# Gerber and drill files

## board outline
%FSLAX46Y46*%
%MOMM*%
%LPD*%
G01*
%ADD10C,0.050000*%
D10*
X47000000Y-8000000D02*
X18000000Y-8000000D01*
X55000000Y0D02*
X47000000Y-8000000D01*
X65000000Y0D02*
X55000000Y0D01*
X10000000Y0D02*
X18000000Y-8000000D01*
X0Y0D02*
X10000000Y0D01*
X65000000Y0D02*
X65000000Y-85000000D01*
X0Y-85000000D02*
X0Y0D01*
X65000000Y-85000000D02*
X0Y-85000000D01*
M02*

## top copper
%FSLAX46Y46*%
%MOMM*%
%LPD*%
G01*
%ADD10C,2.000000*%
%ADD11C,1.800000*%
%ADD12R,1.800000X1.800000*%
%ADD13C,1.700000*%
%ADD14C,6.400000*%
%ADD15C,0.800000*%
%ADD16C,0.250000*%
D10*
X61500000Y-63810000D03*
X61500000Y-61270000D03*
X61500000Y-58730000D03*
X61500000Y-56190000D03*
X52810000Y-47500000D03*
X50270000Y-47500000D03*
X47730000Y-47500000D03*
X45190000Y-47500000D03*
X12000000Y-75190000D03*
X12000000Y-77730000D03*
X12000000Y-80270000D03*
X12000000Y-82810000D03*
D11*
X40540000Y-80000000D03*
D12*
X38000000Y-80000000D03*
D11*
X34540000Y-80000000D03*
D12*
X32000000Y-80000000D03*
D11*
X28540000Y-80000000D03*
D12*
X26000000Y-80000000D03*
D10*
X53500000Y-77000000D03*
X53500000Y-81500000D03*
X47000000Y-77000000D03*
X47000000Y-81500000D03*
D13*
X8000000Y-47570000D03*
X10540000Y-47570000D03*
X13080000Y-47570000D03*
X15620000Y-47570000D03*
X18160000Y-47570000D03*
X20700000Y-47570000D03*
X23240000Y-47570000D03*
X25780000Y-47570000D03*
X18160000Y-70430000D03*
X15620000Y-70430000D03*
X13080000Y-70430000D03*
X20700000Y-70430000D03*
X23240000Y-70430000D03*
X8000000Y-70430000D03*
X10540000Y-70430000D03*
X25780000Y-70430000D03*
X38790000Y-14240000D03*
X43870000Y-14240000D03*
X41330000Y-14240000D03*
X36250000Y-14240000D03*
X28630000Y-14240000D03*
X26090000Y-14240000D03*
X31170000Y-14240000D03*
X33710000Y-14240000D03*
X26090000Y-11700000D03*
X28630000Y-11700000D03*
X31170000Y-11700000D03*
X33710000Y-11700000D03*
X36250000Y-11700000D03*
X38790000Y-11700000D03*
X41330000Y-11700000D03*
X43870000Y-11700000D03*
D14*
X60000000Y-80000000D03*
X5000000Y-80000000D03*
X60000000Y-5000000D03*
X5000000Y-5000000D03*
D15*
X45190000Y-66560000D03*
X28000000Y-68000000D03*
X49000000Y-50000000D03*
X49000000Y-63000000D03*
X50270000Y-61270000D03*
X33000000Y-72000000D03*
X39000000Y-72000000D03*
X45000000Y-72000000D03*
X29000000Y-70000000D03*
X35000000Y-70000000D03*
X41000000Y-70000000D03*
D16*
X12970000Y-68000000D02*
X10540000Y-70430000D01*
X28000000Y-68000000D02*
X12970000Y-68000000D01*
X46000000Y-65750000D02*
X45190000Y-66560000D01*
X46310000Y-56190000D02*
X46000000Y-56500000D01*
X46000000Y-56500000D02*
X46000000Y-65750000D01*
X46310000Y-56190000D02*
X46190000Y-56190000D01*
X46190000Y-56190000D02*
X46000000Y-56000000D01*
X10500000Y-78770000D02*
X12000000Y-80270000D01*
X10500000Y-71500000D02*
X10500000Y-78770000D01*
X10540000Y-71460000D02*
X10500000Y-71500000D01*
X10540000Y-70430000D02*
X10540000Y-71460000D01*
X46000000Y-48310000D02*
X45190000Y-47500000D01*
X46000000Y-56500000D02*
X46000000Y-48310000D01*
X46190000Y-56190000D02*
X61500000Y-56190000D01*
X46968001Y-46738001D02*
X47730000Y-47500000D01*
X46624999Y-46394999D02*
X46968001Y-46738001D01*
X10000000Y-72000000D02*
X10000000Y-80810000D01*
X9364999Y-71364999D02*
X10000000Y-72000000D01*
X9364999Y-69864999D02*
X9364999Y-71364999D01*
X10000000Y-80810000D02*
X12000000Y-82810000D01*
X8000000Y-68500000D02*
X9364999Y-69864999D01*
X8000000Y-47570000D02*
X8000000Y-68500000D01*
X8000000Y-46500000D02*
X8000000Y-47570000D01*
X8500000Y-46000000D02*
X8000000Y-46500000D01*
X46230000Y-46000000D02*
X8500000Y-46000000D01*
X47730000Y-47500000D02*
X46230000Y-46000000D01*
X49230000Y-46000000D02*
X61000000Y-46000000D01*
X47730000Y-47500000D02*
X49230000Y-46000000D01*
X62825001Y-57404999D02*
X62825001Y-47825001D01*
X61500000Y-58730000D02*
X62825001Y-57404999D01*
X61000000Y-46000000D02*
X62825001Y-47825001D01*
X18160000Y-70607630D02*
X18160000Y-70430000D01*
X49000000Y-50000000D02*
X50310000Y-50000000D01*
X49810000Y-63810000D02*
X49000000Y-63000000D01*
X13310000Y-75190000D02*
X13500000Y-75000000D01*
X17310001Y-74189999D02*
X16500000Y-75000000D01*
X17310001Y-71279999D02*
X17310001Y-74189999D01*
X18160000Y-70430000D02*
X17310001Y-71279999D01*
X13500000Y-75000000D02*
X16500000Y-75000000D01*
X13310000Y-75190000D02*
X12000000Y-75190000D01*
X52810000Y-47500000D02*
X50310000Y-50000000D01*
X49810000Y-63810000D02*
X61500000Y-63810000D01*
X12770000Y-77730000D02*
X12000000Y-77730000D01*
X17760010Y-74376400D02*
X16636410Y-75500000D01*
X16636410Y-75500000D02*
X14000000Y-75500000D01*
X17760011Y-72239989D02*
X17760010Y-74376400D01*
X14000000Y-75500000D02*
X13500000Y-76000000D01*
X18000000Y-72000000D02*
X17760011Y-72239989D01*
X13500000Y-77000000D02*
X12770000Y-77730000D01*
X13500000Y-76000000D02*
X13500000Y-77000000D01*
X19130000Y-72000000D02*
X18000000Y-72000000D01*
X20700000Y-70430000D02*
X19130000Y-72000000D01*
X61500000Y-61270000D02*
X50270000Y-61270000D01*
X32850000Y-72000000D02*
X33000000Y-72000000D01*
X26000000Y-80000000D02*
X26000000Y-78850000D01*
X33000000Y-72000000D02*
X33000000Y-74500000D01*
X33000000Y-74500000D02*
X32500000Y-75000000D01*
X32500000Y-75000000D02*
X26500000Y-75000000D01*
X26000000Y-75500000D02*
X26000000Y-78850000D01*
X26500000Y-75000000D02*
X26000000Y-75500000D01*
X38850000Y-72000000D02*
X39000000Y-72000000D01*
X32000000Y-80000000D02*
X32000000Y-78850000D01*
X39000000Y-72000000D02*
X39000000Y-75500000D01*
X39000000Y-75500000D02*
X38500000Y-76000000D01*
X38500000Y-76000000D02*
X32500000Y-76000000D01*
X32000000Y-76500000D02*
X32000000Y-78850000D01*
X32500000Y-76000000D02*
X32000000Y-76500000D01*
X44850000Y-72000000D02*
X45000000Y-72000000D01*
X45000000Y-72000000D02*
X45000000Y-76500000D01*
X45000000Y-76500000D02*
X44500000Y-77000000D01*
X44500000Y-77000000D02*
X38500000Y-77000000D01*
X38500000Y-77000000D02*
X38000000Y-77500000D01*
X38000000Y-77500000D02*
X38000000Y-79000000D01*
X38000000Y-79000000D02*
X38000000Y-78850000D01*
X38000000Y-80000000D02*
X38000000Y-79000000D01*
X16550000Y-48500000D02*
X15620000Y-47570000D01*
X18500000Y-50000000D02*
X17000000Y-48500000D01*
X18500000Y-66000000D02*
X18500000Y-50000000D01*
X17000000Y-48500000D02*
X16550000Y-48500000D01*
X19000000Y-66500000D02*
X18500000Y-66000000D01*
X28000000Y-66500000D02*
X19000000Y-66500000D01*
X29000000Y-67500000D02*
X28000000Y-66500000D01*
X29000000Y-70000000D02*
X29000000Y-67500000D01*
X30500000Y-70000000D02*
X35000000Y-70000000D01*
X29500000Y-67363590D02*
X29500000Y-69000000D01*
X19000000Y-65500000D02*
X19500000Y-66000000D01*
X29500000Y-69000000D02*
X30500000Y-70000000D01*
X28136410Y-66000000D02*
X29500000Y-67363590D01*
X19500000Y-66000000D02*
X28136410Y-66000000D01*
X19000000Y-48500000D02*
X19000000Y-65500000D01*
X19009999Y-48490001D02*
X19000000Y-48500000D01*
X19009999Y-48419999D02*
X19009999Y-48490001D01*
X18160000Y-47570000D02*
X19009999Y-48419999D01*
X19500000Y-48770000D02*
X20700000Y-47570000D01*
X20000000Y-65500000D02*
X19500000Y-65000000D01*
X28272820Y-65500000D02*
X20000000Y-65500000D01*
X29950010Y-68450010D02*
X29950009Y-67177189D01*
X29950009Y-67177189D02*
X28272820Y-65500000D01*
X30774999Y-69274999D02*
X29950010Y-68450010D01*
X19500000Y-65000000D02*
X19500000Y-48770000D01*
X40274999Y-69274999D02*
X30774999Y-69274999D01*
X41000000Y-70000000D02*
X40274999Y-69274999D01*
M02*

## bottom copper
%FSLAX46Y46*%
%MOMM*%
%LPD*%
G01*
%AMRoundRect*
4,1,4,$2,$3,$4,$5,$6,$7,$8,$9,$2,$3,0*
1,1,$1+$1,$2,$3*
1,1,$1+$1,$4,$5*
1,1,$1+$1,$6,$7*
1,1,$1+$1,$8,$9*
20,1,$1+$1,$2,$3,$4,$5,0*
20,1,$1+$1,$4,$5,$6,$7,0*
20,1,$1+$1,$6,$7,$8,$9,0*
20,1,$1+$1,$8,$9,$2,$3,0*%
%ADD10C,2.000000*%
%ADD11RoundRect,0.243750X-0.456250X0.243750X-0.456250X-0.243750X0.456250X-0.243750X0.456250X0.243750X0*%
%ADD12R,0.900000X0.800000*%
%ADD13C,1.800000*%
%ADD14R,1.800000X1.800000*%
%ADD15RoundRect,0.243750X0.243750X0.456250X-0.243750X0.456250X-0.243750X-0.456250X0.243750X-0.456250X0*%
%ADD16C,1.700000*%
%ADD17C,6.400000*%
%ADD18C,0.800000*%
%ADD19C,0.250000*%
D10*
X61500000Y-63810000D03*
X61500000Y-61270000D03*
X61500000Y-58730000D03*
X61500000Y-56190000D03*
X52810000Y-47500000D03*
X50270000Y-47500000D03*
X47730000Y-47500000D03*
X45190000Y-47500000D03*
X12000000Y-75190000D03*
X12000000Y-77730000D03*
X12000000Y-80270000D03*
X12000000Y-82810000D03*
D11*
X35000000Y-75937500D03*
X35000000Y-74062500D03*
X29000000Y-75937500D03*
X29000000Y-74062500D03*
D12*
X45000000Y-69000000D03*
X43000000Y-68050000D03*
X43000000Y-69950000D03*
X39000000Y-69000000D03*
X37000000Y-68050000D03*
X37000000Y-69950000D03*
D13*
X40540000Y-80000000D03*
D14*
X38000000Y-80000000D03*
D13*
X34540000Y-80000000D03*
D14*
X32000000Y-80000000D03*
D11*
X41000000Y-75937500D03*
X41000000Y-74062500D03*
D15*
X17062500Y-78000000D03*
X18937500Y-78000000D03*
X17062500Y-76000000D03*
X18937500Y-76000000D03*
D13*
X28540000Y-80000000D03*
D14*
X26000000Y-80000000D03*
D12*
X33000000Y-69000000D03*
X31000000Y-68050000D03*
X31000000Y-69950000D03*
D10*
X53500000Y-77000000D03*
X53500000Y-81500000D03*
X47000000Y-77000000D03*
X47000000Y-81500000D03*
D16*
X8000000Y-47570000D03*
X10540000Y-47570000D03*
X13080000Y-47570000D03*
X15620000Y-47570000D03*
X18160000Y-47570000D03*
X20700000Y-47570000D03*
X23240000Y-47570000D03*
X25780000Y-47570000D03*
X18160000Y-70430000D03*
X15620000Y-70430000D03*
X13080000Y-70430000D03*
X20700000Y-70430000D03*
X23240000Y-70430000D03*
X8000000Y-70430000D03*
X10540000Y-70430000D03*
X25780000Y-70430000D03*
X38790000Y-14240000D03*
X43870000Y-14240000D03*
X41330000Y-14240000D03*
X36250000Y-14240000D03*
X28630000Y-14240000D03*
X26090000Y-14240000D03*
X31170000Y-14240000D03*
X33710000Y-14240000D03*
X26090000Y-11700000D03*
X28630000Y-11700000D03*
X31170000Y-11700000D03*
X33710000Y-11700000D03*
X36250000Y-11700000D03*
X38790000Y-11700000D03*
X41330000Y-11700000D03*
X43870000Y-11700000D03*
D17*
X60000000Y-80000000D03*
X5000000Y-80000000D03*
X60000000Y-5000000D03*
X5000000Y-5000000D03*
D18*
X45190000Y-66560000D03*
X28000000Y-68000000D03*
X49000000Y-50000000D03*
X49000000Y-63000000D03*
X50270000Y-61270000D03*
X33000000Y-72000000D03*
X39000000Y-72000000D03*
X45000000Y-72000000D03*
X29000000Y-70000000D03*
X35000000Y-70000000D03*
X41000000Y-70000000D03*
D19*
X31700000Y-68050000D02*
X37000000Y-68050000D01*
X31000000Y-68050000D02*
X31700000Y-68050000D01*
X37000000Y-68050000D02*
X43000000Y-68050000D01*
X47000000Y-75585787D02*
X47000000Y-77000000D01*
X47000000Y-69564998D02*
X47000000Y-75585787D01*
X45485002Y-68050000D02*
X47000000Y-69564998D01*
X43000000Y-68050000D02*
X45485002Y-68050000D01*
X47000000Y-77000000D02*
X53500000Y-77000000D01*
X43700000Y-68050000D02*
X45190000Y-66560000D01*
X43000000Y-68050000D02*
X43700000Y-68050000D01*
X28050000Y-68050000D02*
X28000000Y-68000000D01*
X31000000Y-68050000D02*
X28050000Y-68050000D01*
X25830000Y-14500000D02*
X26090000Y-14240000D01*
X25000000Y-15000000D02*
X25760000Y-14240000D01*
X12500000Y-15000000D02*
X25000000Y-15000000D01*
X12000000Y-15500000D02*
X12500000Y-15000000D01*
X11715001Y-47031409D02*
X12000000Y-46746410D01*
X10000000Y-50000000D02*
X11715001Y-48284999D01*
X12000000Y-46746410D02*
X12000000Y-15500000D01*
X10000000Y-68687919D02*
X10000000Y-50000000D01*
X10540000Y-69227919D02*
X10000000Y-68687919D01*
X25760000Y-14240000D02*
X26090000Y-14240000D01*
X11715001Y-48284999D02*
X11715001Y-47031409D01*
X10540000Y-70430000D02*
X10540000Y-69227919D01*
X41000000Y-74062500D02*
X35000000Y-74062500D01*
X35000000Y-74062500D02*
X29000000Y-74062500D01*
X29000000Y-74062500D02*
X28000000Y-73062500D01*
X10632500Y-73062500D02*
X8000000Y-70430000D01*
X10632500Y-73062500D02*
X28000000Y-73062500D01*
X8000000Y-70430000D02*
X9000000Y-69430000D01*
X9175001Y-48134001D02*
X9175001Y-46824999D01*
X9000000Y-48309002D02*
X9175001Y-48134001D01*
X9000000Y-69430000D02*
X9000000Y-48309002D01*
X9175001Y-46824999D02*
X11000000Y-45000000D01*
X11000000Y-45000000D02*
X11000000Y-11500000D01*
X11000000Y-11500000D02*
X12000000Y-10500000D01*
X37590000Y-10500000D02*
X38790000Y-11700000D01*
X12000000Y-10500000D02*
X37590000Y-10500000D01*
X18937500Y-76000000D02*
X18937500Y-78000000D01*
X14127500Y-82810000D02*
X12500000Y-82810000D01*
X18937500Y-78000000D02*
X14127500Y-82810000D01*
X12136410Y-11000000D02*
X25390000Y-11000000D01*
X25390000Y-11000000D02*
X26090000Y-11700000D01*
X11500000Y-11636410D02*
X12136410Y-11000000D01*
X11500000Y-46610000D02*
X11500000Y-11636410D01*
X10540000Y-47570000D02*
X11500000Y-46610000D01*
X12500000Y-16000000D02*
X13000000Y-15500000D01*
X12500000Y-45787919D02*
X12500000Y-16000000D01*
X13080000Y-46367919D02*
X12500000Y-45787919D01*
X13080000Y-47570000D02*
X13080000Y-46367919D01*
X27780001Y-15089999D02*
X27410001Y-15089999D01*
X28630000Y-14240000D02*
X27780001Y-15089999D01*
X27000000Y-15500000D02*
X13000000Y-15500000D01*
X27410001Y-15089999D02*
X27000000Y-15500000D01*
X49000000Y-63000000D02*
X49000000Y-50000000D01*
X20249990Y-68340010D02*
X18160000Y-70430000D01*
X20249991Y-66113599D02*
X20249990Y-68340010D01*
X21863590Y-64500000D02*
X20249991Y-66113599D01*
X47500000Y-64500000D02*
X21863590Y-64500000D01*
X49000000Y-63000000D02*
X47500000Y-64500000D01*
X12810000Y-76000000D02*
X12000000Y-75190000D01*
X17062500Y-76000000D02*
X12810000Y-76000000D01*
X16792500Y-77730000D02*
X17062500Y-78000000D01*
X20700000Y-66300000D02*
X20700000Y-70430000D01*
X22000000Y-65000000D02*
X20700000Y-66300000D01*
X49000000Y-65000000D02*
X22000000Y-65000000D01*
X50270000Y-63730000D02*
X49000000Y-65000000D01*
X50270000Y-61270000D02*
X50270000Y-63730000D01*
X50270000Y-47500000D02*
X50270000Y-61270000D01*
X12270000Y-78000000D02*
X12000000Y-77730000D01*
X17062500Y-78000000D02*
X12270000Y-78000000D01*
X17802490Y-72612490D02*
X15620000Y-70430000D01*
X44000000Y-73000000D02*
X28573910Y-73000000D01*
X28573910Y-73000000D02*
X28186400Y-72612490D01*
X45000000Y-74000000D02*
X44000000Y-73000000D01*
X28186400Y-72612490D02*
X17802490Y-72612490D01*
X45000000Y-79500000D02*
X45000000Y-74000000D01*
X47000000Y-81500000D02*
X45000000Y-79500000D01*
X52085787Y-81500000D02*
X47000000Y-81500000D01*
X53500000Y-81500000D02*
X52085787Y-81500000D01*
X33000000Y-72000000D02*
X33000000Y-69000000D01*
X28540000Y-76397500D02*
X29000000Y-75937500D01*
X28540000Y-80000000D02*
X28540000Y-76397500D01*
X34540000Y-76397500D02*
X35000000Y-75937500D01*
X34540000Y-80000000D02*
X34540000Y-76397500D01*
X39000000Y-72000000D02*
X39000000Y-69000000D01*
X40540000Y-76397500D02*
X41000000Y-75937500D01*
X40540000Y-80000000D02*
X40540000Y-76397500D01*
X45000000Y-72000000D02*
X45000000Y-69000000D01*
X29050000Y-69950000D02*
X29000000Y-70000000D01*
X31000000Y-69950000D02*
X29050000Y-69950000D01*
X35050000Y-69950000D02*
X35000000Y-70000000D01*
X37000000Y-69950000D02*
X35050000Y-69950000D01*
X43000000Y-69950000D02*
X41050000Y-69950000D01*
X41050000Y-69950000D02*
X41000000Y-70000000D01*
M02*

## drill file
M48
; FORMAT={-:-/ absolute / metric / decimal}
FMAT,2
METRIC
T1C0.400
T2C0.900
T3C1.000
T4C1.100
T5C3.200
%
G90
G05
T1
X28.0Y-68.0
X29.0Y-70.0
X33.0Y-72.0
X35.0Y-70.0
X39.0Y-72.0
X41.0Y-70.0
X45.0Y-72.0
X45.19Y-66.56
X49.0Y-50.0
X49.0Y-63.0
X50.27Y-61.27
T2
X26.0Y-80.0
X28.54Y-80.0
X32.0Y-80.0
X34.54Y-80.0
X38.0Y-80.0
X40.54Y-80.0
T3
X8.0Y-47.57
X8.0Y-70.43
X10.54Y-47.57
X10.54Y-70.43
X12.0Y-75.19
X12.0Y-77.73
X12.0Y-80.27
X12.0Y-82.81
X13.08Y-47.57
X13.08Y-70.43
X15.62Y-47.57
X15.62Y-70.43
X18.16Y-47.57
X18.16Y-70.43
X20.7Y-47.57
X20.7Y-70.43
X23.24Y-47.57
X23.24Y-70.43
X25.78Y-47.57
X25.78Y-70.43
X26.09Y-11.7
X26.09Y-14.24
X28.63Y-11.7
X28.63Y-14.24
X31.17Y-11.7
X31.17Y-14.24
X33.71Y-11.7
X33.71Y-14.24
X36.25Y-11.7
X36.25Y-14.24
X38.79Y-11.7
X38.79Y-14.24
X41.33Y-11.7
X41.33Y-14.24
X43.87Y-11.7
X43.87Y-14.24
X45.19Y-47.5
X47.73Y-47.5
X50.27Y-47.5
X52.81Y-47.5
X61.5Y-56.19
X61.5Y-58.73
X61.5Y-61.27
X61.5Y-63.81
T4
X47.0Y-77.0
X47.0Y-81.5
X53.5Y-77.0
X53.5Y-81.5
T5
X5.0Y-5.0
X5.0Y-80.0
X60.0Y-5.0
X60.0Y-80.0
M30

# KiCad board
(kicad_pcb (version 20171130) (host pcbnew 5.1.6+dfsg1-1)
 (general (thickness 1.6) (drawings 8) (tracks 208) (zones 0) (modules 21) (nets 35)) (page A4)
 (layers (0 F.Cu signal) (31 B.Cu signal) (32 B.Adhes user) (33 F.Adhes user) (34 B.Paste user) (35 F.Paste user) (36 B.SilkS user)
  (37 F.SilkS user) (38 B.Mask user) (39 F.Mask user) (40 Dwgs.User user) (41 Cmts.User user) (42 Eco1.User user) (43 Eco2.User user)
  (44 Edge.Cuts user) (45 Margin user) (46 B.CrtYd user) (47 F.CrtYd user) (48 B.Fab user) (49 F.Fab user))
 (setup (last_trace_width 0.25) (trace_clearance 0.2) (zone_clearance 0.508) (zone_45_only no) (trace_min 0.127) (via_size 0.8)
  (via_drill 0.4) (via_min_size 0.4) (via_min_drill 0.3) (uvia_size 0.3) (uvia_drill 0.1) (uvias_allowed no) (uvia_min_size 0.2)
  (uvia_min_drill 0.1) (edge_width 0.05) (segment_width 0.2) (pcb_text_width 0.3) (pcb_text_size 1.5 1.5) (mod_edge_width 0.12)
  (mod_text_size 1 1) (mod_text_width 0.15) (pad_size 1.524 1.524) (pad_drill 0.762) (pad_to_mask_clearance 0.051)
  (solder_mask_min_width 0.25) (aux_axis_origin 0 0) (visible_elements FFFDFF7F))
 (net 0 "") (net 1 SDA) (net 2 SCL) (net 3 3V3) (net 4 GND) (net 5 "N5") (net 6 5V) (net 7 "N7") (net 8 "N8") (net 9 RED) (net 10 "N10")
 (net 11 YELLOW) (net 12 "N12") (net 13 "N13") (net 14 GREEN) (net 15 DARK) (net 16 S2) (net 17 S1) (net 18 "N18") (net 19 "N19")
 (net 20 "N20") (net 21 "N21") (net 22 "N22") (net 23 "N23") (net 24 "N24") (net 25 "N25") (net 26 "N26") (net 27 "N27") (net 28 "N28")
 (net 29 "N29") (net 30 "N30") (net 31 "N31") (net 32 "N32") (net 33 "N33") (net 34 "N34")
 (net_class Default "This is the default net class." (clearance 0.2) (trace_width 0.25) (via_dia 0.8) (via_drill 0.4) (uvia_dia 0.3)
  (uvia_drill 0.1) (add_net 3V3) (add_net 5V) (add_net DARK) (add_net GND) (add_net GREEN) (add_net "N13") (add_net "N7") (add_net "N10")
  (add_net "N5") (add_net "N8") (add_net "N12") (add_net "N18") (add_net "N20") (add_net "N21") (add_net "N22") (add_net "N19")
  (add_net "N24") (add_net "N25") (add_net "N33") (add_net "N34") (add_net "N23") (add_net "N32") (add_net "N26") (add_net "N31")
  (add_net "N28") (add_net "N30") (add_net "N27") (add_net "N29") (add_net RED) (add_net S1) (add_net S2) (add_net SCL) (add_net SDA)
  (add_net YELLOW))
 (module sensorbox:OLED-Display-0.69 (layer F.Cu) (at 49 60 270)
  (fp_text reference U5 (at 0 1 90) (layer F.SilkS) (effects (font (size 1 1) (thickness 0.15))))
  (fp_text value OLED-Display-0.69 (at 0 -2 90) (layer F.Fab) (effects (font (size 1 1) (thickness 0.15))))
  (pad 4 thru_hole circle (at 3.81 -12.5 270) (size 2 2) (drill 1) (layers *.Cu *.Mask) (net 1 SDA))
  (pad 3 thru_hole circle (at 1.27 -12.5 270) (size 2 2) (drill 1) (layers *.Cu *.Mask) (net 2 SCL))
  (pad 2 thru_hole circle (at -1.27 -12.5 270) (size 2 2) (drill 1) (layers *.Cu *.Mask) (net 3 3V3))
  (pad 1 thru_hole circle (at -3.81 -12.5 270) (size 2 2) (drill 1) (layers *.Cu *.Mask) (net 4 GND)))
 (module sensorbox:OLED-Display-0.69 (layer F.Cu) (at 49 60)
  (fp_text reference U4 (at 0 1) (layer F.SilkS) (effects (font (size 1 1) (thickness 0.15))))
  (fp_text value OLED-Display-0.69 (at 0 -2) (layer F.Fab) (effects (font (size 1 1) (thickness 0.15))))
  (pad 4 thru_hole circle (at 3.81 -12.5) (size 2 2) (drill 1) (layers *.Cu *.Mask) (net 1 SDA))
  (pad 3 thru_hole circle (at 1.27 -12.5) (size 2 2) (drill 1) (layers *.Cu *.Mask) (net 2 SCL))
  (pad 2 thru_hole circle (at -1.27 -12.5) (size 2 2) (drill 1) (layers *.Cu *.Mask) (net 3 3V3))
  (pad 1 thru_hole circle (at -3.81 -12.5) (size 2 2) (drill 1) (layers *.Cu *.Mask) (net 4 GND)))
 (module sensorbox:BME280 (layer F.Cu) (at 16.5 79 90)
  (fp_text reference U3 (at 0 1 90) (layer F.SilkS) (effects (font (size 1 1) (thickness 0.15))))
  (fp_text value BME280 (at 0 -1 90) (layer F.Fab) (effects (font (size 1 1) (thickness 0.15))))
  (pad 4 thru_hole circle (at 3.81 -4.5 90) (size 2 2) (drill 1) (layers *.Cu *.Mask) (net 1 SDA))
  (pad 3 thru_hole circle (at 1.27 -4.5 90) (size 2 2) (drill 1) (layers *.Cu *.Mask) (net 2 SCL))
  (pad 2 thru_hole circle (at -1.27 -4.5 90) (size 2 2) (drill 1) (layers *.Cu *.Mask) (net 4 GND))
  (pad 1 thru_hole circle (at -3.81 -4.5 90) (size 2 2) (drill 1) (layers *.Cu *.Mask) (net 3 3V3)))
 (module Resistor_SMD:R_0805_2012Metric (layer B.Cu) (at 35 75 270)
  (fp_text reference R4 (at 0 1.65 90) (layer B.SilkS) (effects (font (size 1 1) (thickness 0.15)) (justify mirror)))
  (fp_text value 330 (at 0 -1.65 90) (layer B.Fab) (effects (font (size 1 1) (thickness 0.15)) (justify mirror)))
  (pad 2 smd roundrect (at 0.9375 0 270) (size 0.975 1.4) (layers B.Cu B.Paste B.Mask) (roundrect_rratio 0.25) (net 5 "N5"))
  (pad 1 smd roundrect (at -0.9375 0 270) (size 0.975 1.4) (layers B.Cu B.Paste B.Mask) (roundrect_rratio 0.25) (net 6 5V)))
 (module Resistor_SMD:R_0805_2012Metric (layer B.Cu) (at 29 75 270)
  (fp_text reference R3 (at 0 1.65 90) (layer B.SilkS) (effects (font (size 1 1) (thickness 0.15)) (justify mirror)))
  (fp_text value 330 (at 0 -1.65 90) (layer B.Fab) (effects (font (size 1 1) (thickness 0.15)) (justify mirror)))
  (pad 2 smd roundrect (at 0.9375 0 270) (size 0.975 1.4) (layers B.Cu B.Paste B.Mask) (roundrect_rratio 0.25) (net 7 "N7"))
  (pad 1 smd roundrect (at -0.9375 0 270) (size 0.975 1.4) (layers B.Cu B.Paste B.Mask) (roundrect_rratio 0.25) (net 6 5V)))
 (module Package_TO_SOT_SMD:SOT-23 (layer B.Cu) (at 44 69)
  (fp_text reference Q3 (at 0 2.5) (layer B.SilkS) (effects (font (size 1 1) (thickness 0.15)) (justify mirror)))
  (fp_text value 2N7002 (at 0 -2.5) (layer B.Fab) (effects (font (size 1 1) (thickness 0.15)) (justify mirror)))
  (pad 3 smd rect (at 1 0) (size 0.9 0.8) (layers B.Cu B.Paste B.Mask) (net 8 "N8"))
  (pad 2 smd rect (at -1 -0.95) (size 0.9 0.8) (layers B.Cu B.Paste B.Mask) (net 4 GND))
  (pad 1 smd rect (at -1 0.95) (size 0.9 0.8) (layers B.Cu B.Paste B.Mask) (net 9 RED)))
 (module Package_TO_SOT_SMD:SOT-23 (layer B.Cu) (at 38 69)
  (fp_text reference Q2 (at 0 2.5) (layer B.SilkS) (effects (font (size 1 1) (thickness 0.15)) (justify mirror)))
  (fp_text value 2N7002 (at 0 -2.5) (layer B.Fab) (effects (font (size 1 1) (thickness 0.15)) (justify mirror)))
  (pad 3 smd rect (at 1 0) (size 0.9 0.8) (layers B.Cu B.Paste B.Mask) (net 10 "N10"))
  (pad 2 smd rect (at -1 -0.95) (size 0.9 0.8) (layers B.Cu B.Paste B.Mask) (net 4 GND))
  (pad 1 smd rect (at -1 0.95) (size 0.9 0.8) (layers B.Cu B.Paste B.Mask) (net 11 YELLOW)))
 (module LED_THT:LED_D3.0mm (layer F.Cu) (at 38 80)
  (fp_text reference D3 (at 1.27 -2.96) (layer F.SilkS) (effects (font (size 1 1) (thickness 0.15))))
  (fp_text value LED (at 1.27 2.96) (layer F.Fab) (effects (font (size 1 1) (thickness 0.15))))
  (pad 2 thru_hole circle (at 2.54 0) (size 1.8 1.8) (drill 0.9) (layers *.Cu *.Mask) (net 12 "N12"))
  (pad 1 thru_hole rect (at 0 0) (size 1.8 1.8) (drill 0.9) (layers *.Cu *.Mask) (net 8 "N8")))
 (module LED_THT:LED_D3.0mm (layer F.Cu) (at 32 80)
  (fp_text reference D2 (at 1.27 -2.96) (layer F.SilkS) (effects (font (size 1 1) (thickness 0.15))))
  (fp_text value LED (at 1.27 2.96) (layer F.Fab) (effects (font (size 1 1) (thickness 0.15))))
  (pad 2 thru_hole circle (at 2.54 0) (size 1.8 1.8) (drill 0.9) (layers *.Cu *.Mask) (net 5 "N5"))
  (pad 1 thru_hole rect (at 0 0) (size 1.8 1.8) (drill 0.9) (layers *.Cu *.Mask) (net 10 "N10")))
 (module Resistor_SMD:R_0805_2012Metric (layer B.Cu) (at 41 75 270)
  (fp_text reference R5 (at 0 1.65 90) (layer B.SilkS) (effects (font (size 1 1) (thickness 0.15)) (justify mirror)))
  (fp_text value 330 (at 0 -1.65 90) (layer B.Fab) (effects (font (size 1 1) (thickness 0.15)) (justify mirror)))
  (pad 2 smd roundrect (at 0.9375 0 270) (size 0.975 1.4) (layers B.Cu B.Paste B.Mask) (roundrect_rratio 0.25) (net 12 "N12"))
  (pad 1 smd roundrect (at -0.9375 0 270) (size 0.975 1.4) (layers B.Cu B.Paste B.Mask) (roundrect_rratio 0.25) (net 6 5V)))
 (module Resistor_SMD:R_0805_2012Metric (layer B.Cu) (at 18 78 180)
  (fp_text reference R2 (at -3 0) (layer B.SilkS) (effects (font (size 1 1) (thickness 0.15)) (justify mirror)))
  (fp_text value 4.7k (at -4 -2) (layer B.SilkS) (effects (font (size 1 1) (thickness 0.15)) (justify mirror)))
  (pad 2 smd roundrect (at 0.9375 0 180) (size 0.975 1.4) (layers B.Cu B.Paste B.Mask) (roundrect_rratio 0.25) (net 2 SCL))
  (pad 1 smd roundrect (at -0.9375 0 180) (size 0.975 1.4) (layers B.Cu B.Paste B.Mask) (roundrect_rratio 0.25) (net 3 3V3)))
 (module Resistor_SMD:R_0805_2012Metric (layer B.Cu) (at 18 76 180)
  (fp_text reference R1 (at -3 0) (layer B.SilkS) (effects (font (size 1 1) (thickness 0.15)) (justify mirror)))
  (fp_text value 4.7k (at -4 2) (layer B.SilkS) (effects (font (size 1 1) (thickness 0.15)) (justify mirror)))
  (pad 2 smd roundrect (at 0.9375 0 180) (size 0.975 1.4) (layers B.Cu B.Paste B.Mask) (roundrect_rratio 0.25) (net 1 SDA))
  (pad 1 smd roundrect (at -0.9375 0 180) (size 0.975 1.4) (layers B.Cu B.Paste B.Mask) (roundrect_rratio 0.25) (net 3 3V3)))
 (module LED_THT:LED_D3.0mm (layer F.Cu) (at 26 80)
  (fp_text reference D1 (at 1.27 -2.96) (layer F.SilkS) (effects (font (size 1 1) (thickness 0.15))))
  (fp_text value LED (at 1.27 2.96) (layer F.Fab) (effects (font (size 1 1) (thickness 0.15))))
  (pad 2 thru_hole circle (at 2.54 0) (size 1.8 1.8) (drill 0.9) (layers *.Cu *.Mask) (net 7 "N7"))
  (pad 1 thru_hole rect (at 0 0) (size 1.8 1.8) (drill 0.9) (layers *.Cu *.Mask) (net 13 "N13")))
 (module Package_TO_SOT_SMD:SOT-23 (layer B.Cu) (at 32 69)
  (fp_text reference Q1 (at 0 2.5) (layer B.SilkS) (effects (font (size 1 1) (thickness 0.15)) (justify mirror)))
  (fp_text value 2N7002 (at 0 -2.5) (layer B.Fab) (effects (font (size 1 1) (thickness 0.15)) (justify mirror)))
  (pad 3 smd rect (at 1 0) (size 0.9 0.8) (layers B.Cu B.Paste B.Mask) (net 13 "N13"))
  (pad 2 smd rect (at -1 -0.95) (size 0.9 0.8) (layers B.Cu B.Paste B.Mask) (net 4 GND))
  (pad 1 smd rect (at -1 0.95) (size 0.9 0.8) (layers B.Cu B.Paste B.Mask) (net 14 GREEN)))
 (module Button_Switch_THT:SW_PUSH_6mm (layer F.Cu) (at 47 77)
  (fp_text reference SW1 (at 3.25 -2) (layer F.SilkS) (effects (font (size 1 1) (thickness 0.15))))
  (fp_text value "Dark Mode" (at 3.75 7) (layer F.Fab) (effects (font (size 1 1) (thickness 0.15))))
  (pad 1 thru_hole circle (at 6.5 0 90) (size 2 2) (drill 1.1) (layers *.Cu *.Mask) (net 4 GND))
  (pad 2 thru_hole circle (at 6.5 4.5 90) (size 2 2) (drill 1.1) (layers *.Cu *.Mask) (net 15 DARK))
  (pad 1 thru_hole circle (at 0 0 90) (size 2 2) (drill 1.1) (layers *.Cu *.Mask) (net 4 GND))
  (pad 2 thru_hole circle (at 0 4.5 90) (size 2 2) (drill 1.1) (layers *.Cu *.Mask) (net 15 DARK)))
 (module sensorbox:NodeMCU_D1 (layer F.Cu) (at -1 59)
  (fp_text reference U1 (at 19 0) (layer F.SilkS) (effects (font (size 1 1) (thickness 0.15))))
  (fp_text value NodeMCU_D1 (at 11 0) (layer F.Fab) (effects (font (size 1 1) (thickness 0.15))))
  (pad 16 thru_hole circle (at 9 -11.43) (size 1.7 1.7) (drill 1) (layers *.Cu *.Mask) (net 3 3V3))
  (pad 15 thru_hole circle (at 11.54 -11.43) (size 1.7 1.7) (drill 1) (layers *.Cu *.Mask) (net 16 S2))
  (pad 14 thru_hole circle (at 14.08 -11.43) (size 1.7 1.7) (drill 1) (layers *.Cu *.Mask) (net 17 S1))
  (pad 13 thru_hole circle (at 16.62 -11.43) (size 1.7 1.7) (drill 1) (layers *.Cu *.Mask) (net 14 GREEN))
  (pad 12 thru_hole circle (at 19.16 -11.43) (size 1.7 1.7) (drill 1) (layers *.Cu *.Mask) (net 11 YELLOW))
  (pad 11 thru_hole circle (at 21.7 -11.43) (size 1.7 1.7) (drill 1) (layers *.Cu *.Mask) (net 9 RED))
  (pad 10 thru_hole circle (at 24.24 -11.43) (size 1.7 1.7) (drill 1) (layers *.Cu *.Mask) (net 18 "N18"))
  (pad 9 thru_hole circle (at 26.78 -11.43) (size 1.7 1.7) (drill 1) (layers *.Cu *.Mask) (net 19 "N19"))
  (pad 5 thru_hole circle (at 19.16 11.43) (size 1.7 1.7) (drill 1) (layers *.Cu *.Mask) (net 1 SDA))
  (pad 4 thru_hole circle (at 16.62 11.43) (size 1.7 1.7) (drill 1) (layers *.Cu *.Mask) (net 15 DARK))
  (pad 3 thru_hole circle (at 14.08 11.43) (size 1.7 1.7) (drill 1) (layers *.Cu *.Mask) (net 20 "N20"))
  (pad 6 thru_hole circle (at 21.7 11.43) (size 1.7 1.7) (drill 1) (layers *.Cu *.Mask) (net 2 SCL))
  (pad 7 thru_hole circle (at 24.24 11.43) (size 1.7 1.7) (drill 1) (layers *.Cu *.Mask) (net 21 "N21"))
  (pad 1 thru_hole circle (at 9 11.43) (size 1.7 1.7) (drill 1) (layers *.Cu *.Mask) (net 6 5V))
  (pad 2 thru_hole circle (at 11.54 11.43) (size 1.7 1.7) (drill 1) (layers *.Cu *.Mask) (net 4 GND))
  (pad 8 thru_hole circle (at 26.78 11.43) (size 1.7 1.7) (drill 1) (layers *.Cu *.Mask) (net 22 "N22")))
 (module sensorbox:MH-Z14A (layer F.Cu) (at 61 44 180)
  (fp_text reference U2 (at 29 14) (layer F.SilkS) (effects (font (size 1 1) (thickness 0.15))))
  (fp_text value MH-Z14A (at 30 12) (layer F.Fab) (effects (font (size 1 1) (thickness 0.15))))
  (pad 2 thru_hole circle (at 22.21 29.76 180) (size 1.7 1.7) (drill 1) (layers *.Cu *.Mask) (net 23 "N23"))
  (pad 14 thru_hole circle (at 17.13 29.76 180) (size 1.7 1.7) (drill 1) (layers *.Cu *.Mask) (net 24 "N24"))
  (pad 15 thru_hole circle (at 19.67 29.76 180) (size 1.7 1.7) (drill 1) (layers *.Cu *.Mask) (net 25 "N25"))
  (pad 4 thru_hole circle (at 24.75 29.76 180) (size 1.7 1.7) (drill 1) (layers *.Cu *.Mask) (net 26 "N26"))
  (pad 10 thru_hole circle (at 32.37 29.76 180) (size 1.7 1.7) (drill 1) (layers *.Cu *.Mask) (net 17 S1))
  (pad 12 thru_hole circle (at 34.91 29.76 180) (size 1.7 1.7) (drill 1) (layers *.Cu *.Mask) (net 4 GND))
  (pad 8 thru_hole circle (at 29.83 29.76 180) (size 1.7 1.7) (drill 1) (layers *.Cu *.Mask) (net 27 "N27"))
  (pad 6 thru_hole circle (at 27.29 29.76 180) (size 1.7 1.7) (drill 1) (layers *.Cu *.Mask) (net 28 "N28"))
  (pad 11 thru_hole circle (at 34.91 32.3 180) (size 1.7 1.7) (drill 1) (layers *.Cu *.Mask) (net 16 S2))
  (pad 9 thru_hole circle (at 32.37 32.3 180) (size 1.7 1.7) (drill 1) (layers *.Cu *.Mask) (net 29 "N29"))
  (pad 7 thru_hole circle (at 29.83 32.3 180) (size 1.7 1.7) (drill 1) (layers *.Cu *.Mask) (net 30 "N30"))
  (pad 5 thru_hole circle (at 27.29 32.3 180) (size 1.7 1.7) (drill 1) (layers *.Cu *.Mask) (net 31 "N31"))
  (pad 3 thru_hole circle (at 24.75 32.3 180) (size 1.7 1.7) (drill 1) (layers *.Cu *.Mask) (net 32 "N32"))
  (pad 1 thru_hole circle (at 22.21 32.3 180) (size 1.7 1.7) (drill 1) (layers *.Cu *.Mask) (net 6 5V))
  (pad 16 thru_hole circle (at 19.67 32.3 180) (size 1.7 1.7) (drill 1) (layers *.Cu *.Mask) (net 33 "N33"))
  (pad 17 thru_hole circle (at 17.13 32.3 180) (size 1.7 1.7) (drill 1) (layers *.Cu *.Mask) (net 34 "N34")))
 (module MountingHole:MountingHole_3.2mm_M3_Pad (layer F.Cu) (at 60 80)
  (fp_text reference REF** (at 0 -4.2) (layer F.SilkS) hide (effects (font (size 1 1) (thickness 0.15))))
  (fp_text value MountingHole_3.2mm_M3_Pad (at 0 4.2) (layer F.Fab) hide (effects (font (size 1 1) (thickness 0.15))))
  (pad 1 thru_hole circle (at 0 0) (size 6.4 6.4) (drill 3.2) (layers *.Cu *.Mask)))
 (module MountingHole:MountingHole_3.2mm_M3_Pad (layer F.Cu) (at 5 80)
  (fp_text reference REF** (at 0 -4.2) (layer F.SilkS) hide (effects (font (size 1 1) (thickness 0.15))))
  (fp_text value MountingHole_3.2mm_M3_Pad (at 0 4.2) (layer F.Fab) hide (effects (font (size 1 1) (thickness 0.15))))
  (pad 1 thru_hole circle (at 0 0) (size 6.4 6.4) (drill 3.2) (layers *.Cu *.Mask)))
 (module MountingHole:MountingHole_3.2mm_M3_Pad (layer F.Cu) (at 60 5)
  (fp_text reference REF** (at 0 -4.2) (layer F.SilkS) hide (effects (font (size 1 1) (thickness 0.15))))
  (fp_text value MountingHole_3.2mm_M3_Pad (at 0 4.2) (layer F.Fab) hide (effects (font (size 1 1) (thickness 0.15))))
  (pad 1 thru_hole circle (at 0 0) (size 6.4 6.4) (drill 3.2) (layers *.Cu *.Mask)))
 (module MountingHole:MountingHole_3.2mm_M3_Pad (layer F.Cu) (at 5 5)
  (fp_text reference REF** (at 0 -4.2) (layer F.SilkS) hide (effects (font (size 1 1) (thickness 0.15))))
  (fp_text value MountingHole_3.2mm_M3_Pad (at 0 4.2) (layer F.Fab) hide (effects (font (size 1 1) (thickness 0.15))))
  (pad 1 thru_hole circle (at 0 0) (size 6.4 6.4) (drill 3.2) (layers *.Cu *.Mask)))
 (gr_line (start 47 8) (end 18 8) (layer Edge.Cuts) (width 0.05))
 (gr_line (start 55 0) (end 47 8) (layer Edge.Cuts) (width 0.05))
 (gr_line (start 65 0) (end 55 0) (layer Edge.Cuts) (width 0.05))
 (gr_line (start 10 0) (end 18 8) (layer Edge.Cuts) (width 0.05))
 (gr_line (start 0 0) (end 10 0) (layer Edge.Cuts) (width 0.05))
 (gr_line (start 65 0) (end 65 85) (layer Edge.Cuts) (width 0.05))
 (gr_line (start 0 85) (end 0 0) (layer Edge.Cuts) (width 0.05))
 (gr_line (start 65 85) (end 0 85) (layer Edge.Cuts) (width 0.05))
 (segment (start 31.7 68.05) (end 37 68.05) (width 0.25) (layer B.Cu) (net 4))
 (segment (start 31 68.05) (end 31.7 68.05) (width 0.25) (layer B.Cu) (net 4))
 (segment (start 37 68.05) (end 43 68.05) (width 0.25) (layer B.Cu) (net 4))
 (segment (start 47 75.585787) (end 47 77) (width 0.25) (layer B.Cu) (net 4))
 (segment (start 47 69.564998) (end 47 75.585787) (width 0.25) (layer B.Cu) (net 4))
 (segment (start 45.485002 68.05) (end 47 69.564998) (width 0.25) (layer B.Cu) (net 4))
 (segment (start 43 68.05) (end 45.485002 68.05) (width 0.25) (layer B.Cu) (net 4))
 (segment (start 47 77) (end 53.5 77) (width 0.25) (layer B.Cu) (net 4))
 (segment (start 43.7 68.05) (end 45.19 66.56) (width 0.25) (layer B.Cu) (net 4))
 (segment (start 43 68.05) (end 43.7 68.05) (width 0.25) (layer B.Cu) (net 4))
 (via (at 45.19 66.56) (size 0.8) (drill 0.4) (layers F.Cu B.Cu) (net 4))
 (via (at 28 68) (size 0.8) (drill 0.4) (layers F.Cu B.Cu) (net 4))
 (segment (start 28.05 68.05) (end 28 68) (width 0.25) (layer B.Cu) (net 4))
 (segment (start 31 68.05) (end 28.05 68.05) (width 0.25) (layer B.Cu) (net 4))
 (segment (start 12.97 68) (end 10.54 70.43) (width 0.25) (layer F.Cu) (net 4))
 (segment (start 28 68) (end 12.97 68) (width 0.25) (layer F.Cu) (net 4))
 (segment (start 46 65.75) (end 45.19 66.56) (width 0.25) (layer F.Cu) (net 4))
 (segment (start 25.83 14.5) (end 26.09 14.24) (width 0.25) (layer B.Cu) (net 4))
 (segment (start 46.31 56.19) (end 46 56.5) (width 0.25) (layer F.Cu) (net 4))
 (segment (start 46 56.5) (end 46 65.75) (width 0.25) (layer F.Cu) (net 4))
 (segment (start 46.31 56.19) (end 46.19 56.19) (width 0.25) (layer F.Cu) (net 4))
 (segment (start 46.19 56.19) (end 46 56) (width 0.25) (layer F.Cu) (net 4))
 (segment (start 25 15) (end 25.76 14.24) (width 0.25) (layer B.Cu) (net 4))
 (segment (start 12.5 15) (end 25 15) (width 0.25) (layer B.Cu) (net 4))
 (segment (start 12 15.5) (end 12.5 15) (width 0.25) (layer B.Cu) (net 4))
 (segment (start 11.715001 47.031409) (end 12 46.74641) (width 0.25) (layer B.Cu) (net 4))
 (segment (start 10 50) (end 11.715001 48.284999) (width 0.25) (layer B.Cu) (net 4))
 (segment (start 12 46.74641) (end 12 15.5) (width 0.25) (layer B.Cu) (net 4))
 (segment (start 10 68.687919) (end 10 50) (width 0.25) (layer B.Cu) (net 4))
 (segment (start 10.54 69.227919) (end 10 68.687919) (width 0.25) (layer B.Cu) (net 4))
 (segment (start 25.76 14.24) (end 26.09 14.24) (width 0.25) (layer B.Cu) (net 4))
 (segment (start 11.715001 48.284999) (end 11.715001 47.031409) (width 0.25) (layer B.Cu) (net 4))
 (segment (start 10.54 70.43) (end 10.54 69.227919) (width 0.25) (layer B.Cu) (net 4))
 (segment (start 10.5 78.77) (end 12 80.27) (width 0.25) (layer F.Cu) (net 4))
 (segment (start 10.5 71.5) (end 10.5 78.77) (width 0.25) (layer F.Cu) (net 4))
 (segment (start 10.54 71.46) (end 10.5 71.5) (width 0.25) (layer F.Cu) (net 4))
 (segment (start 10.54 70.43) (end 10.54 71.46) (width 0.25) (layer F.Cu) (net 4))
 (segment (start 46 48.31) (end 45.19 47.5) (width 0.25) (layer F.Cu) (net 4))
 (segment (start 46 56.5) (end 46 48.31) (width 0.25) (layer F.Cu) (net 4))
 (segment (start 46.19 56.19) (end 61.5 56.19) (width 0.25) (layer F.Cu) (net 4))
 (segment (start 41 74.0625) (end 35 74.0625) (width 0.25) (layer B.Cu) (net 6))
 (segment (start 35 74.0625) (end 29 74.0625) (width 0.25) (layer B.Cu) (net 6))
 (segment (start 29 74.0625) (end 28 73.0625) (width 0.25) (layer B.Cu) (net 6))
 (segment (start 10.6325 73.0625) (end 8 70.43) (width 0.25) (layer B.Cu) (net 6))
 (segment (start 10.6325 73.0625) (end 28 73.0625) (width 0.25) (layer B.Cu) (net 6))
 (segment (start 8 70.43) (end 9 69.43) (width 0.25) (layer B.Cu) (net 6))
 (segment (start 9.175001 48.134001) (end 9.175001 46.824999) (width 0.25) (layer B.Cu) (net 6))
 (segment (start 9 48.309002) (end 9.175001 48.134001) (width 0.25) (layer B.Cu) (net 6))
 (segment (start 9 69.43) (end 9 48.309002) (width 0.25) (layer B.Cu) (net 6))
 (segment (start 9.175001 46.824999) (end 11 45) (width 0.25) (layer B.Cu) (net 6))
 (segment (start 11 45) (end 11 11.5) (width 0.25) (layer B.Cu) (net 6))
 (segment (start 11 11.5) (end 12 10.5) (width 0.25) (layer B.Cu) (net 6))
 (segment (start 37.59 10.5) (end 38.79 11.7) (width 0.25) (layer B.Cu) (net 6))
 (segment (start 12 10.5) (end 37.59 10.5) (width 0.25) (layer B.Cu) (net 6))
 (segment (start 18.9375 76) (end 18.9375 78) (width 0.25) (layer B.Cu) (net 3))
 (segment (start 14.1275 82.81) (end 12.5 82.81) (width 0.25) (layer B.Cu) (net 3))
 (segment (start 18.9375 78) (end 14.1275 82.81) (width 0.25) (layer B.Cu) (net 3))
 (segment (start 46.968001 46.738001) (end 47.73 47.5) (width 0.25) (layer F.Cu) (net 3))
 (segment (start 46.624999 46.394999) (end 46.968001 46.738001) (width 0.25) (layer F.Cu) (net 3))
 (segment (start 10 72) (end 10 80.81) (width 0.25) (layer F.Cu) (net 3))
 (segment (start 9.364999 71.364999) (end 10 72) (width 0.25) (layer F.Cu) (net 3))
 (segment (start 9.364999 69.864999) (end 9.364999 71.364999) (width 0.25) (layer F.Cu) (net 3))
 (segment (start 10 80.81) (end 12 82.81) (width 0.25) (layer F.Cu) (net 3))
 (segment (start 8 68.5) (end 9.364999 69.864999) (width 0.25) (layer F.Cu) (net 3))
 (segment (start 8 47.57) (end 8 68.5) (width 0.25) (layer F.Cu) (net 3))
 (segment (start 8 46.5) (end 8 47.57) (width 0.25) (layer F.Cu) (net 3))
 (segment (start 8.5 46) (end 8 46.5) (width 0.25) (layer F.Cu) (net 3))
 (segment (start 46.23 46) (end 8.5 46) (width 0.25) (layer F.Cu) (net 3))
 (segment (start 47.73 47.5) (end 46.23 46) (width 0.25) (layer F.Cu) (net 3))
 (segment (start 49.23 46) (end 61 46) (width 0.25) (layer F.Cu) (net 3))
 (segment (start 47.73 47.5) (end 49.23 46) (width 0.25) (layer F.Cu) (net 3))
 (segment (start 62.825001 57.404999) (end 62.825001 47.825001) (width 0.25) (layer F.Cu) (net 3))
 (segment (start 61.5 58.73) (end 62.825001 57.404999) (width 0.25) (layer F.Cu) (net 3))
 (segment (start 61 46) (end 62.825001 47.825001) (width 0.25) (layer F.Cu) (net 3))
 (segment (start 12.13641 11) (end 25.39 11) (width 0.25) (layer B.Cu) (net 16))
 (segment (start 25.39 11) (end 26.09 11.7) (width 0.25) (layer B.Cu) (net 16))
 (segment (start 11.5 11.63641) (end 12.13641 11) (width 0.25) (layer B.Cu) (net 16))
 (segment (start 11.5 46.61) (end 11.5 11.63641) (width 0.25) (layer B.Cu) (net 16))
 (segment (start 10.54 47.57) (end 11.5 46.61) (width 0.25) (layer B.Cu) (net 16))
 (segment (start 12.5 16) (end 13 15.5) (width 0.25) (layer B.Cu) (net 17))
 (segment (start 12.5 45.787919) (end 12.5 16) (width 0.25) (layer B.Cu) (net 17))
 (segment (start 13.08 46.367919) (end 12.5 45.787919) (width 0.25) (layer B.Cu) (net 17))
 (segment (start 13.08 47.57) (end 13.08 46.367919) (width 0.25) (layer B.Cu) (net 17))
 (segment (start 27.780001 15.089999) (end 27.410001 15.089999) (width 0.25) (layer B.Cu) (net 17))
 (segment (start 28.63 14.24) (end 27.780001 15.089999) (width 0.25) (layer B.Cu) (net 17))
 (segment (start 27 15.5) (end 13 15.5) (width 0.25) (layer B.Cu) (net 17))
 (segment (start 27.410001 15.089999) (end 27 15.5) (width 0.25) (layer B.Cu) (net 17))
 (segment (start 18.16 70.60763) (end 18.16 70.43) (width 0.25) (layer F.Cu) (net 1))
 (segment (start 49 63) (end 49 50) (width 0.25) (layer B.Cu) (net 1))
 (via (at 49 50) (size 0.8) (drill 0.4) (layers F.Cu B.Cu) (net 1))
 (segment (start 49 50) (end 50.31 50) (width 0.25) (layer F.Cu) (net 1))
 (via (at 49 63) (size 0.8) (drill 0.4) (layers F.Cu B.Cu) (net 1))
 (segment (start 49.81 63.81) (end 49 63) (width 0.25) (layer F.Cu) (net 1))
 (segment (start 13.31 75.19) (end 13.5 75) (width 0.25) (layer F.Cu) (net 1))
 (segment (start 17.310001 74.189999) (end 16.5 75) (width 0.25) (layer F.Cu) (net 1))
 (segment (start 17.310001 71.279999) (end 17.310001 74.189999) (width 0.25) (layer F.Cu) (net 1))
 (segment (start 18.16 70.43) (end 17.310001 71.279999) (width 0.25) (layer F.Cu) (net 1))
 (segment (start 13.5 75) (end 16.5 75) (width 0.25) (layer F.Cu) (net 1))
 (segment (start 20.24999 68.34001) (end 18.16 70.43) (width 0.25) (layer B.Cu) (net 1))
 (segment (start 20.249991 66.113599) (end 20.24999 68.34001) (width 0.25) (layer B.Cu) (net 1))
 (segment (start 21.86359 64.5) (end 20.249991 66.113599) (width 0.25) (layer B.Cu) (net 1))
 (segment (start 47.5 64.5) (end 21.86359 64.5) (width 0.25) (layer B.Cu) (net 1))
 (segment (start 49 63) (end 47.5 64.5) (width 0.25) (layer B.Cu) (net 1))
 (segment (start 13.31 75.19) (end 12 75.19) (width 0.25) (layer F.Cu) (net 1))
 (segment (start 12.81 76) (end 12 75.19) (width 0.25) (layer B.Cu) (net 1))
 (segment (start 17.0625 76) (end 12.81 76) (width 0.25) (layer B.Cu) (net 1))
 (segment (start 52.81 47.5) (end 50.31 50) (width 0.25) (layer F.Cu) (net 1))
 (segment (start 49.81 63.81) (end 61.5 63.81) (width 0.25) (layer F.Cu) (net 1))
 (segment (start 16.7925 77.73) (end 17.0625 78) (width 0.25) (layer B.Cu) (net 2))
 (segment (start 20.7 66.3) (end 20.7 70.43) (width 0.25) (layer B.Cu) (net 2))
 (segment (start 22 65) (end 20.7 66.3) (width 0.25) (layer B.Cu) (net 2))
 (segment (start 49 65) (end 22 65) (width 0.25) (layer B.Cu) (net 2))
 (segment (start 50.27 63.73) (end 49 65) (width 0.25) (layer B.Cu) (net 2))
 (segment (start 12.77 77.73) (end 12 77.73) (width 0.25) (layer F.Cu) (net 2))
 (segment (start 17.76001 74.3764) (end 16.63641 75.5) (width 0.25) (layer F.Cu) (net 2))
 (segment (start 16.63641 75.5) (end 14 75.5) (width 0.25) (layer F.Cu) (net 2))
 (segment (start 17.760011 72.239989) (end 17.76001 74.3764) (width 0.25) (layer F.Cu) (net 2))
 (segment (start 14 75.5) (end 13.5 76) (width 0.25) (layer F.Cu) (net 2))
 (segment (start 18 72) (end 17.760011 72.239989) (width 0.25) (layer F.Cu) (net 2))
 (segment (start 13.5 77) (end 12.77 77.73) (width 0.25) (layer F.Cu) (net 2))
 (segment (start 13.5 76) (end 13.5 77) (width 0.25) (layer F.Cu) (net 2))
 (segment (start 19.13 72) (end 18 72) (width 0.25) (layer F.Cu) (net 2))
 (segment (start 20.7 70.43) (end 19.13 72) (width 0.25) (layer F.Cu) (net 2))
 (segment (start 50.27 61.27) (end 50.27 63.73) (width 0.25) (layer B.Cu) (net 2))
 (segment (start 50.27 47.5) (end 50.27 61.27) (width 0.25) (layer B.Cu) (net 2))
 (via (at 50.27 61.27) (size 0.8) (drill 0.4) (layers F.Cu B.Cu) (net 2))
 (segment (start 61.5 61.27) (end 50.27 61.27) (width 0.25) (layer F.Cu) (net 2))
 (segment (start 12.27 78) (end 12 77.73) (width 0.25) (layer B.Cu) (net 2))
 (segment (start 17.0625 78) (end 12.27 78) (width 0.25) (layer B.Cu) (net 2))
 (segment (start 17.80249 72.61249) (end 15.62 70.43) (width 0.25) (layer B.Cu) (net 15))
 (segment (start 44 73) (end 28.57391 73) (width 0.25) (layer B.Cu) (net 15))
 (segment (start 28.57391 73) (end 28.1864 72.61249) (width 0.25) (layer B.Cu) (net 15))
 (segment (start 45 74) (end 44 73) (width 0.25) (layer B.Cu) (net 15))
 (segment (start 28.1864 72.61249) (end 17.80249 72.61249) (width 0.25) (layer B.Cu) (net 15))
 (segment (start 45 79.5) (end 45 74) (width 0.25) (layer B.Cu) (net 15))
 (segment (start 47 81.5) (end 45 79.5) (width 0.25) (layer B.Cu) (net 15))
 (segment (start 52.085787 81.5) (end 47 81.5) (width 0.25) (layer B.Cu) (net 15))
 (segment (start 53.5 81.5) (end 52.085787 81.5) (width 0.25) (layer B.Cu) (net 15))
 (via (at 33 72) (size 0.8) (drill 0.4) (layers F.Cu B.Cu) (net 13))
 (segment (start 32.85 72) (end 33 72) (width 0.25) (layer F.Cu) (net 13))
 (segment (start 26 80) (end 26 78.85) (width 0.25) (layer F.Cu) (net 13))
 (segment (start 33 72) (end 33 69) (width 0.25) (layer B.Cu) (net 13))
 (segment (start 33 72) (end 33 74.5) (width 0.25) (layer F.Cu) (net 13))
 (segment (start 33 74.5) (end 32.5 75) (width 0.25) (layer F.Cu) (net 13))
 (segment (start 32.5 75) (end 26.5 75) (width 0.25) (layer F.Cu) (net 13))
 (segment (start 26 75.5) (end 26 78.85) (width 0.25) (layer F.Cu) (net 13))
 (segment (start 26.5 75) (end 26 75.5) (width 0.25) (layer F.Cu) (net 13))
 (segment (start 28.54 76.3975) (end 29 75.9375) (width 0.25) (layer B.Cu) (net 7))
 (segment (start 28.54 80) (end 28.54 76.3975) (width 0.25) (layer B.Cu) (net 7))
 (segment (start 34.54 76.3975) (end 35 75.9375) (width 0.25) (layer B.Cu) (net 5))
 (segment (start 34.54 80) (end 34.54 76.3975) (width 0.25) (layer B.Cu) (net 5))
 (via (at 39 72) (size 0.8) (drill 0.4) (layers F.Cu B.Cu) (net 10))
 (segment (start 38.85 72) (end 39 72) (width 0.25) (layer F.Cu) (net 10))
 (segment (start 32 80) (end 32 78.85) (width 0.25) (layer F.Cu) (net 10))
 (segment (start 39 72) (end 39 69) (width 0.25) (layer B.Cu) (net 10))
 (segment (start 39 72) (end 39 75.5) (width 0.25) (layer F.Cu) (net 10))
 (segment (start 39 75.5) (end 38.5 76) (width 0.25) (layer F.Cu) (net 10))
 (segment (start 38.5 76) (end 32.5 76) (width 0.25) (layer F.Cu) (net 10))
 (segment (start 32 76.5) (end 32 78.85) (width 0.25) (layer F.Cu) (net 10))
 (segment (start 32.5 76) (end 32 76.5) (width 0.25) (layer F.Cu) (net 10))
 (segment (start 40.54 76.3975) (end 41 75.9375) (width 0.25) (layer B.Cu) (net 12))
 (segment (start 40.54 80) (end 40.54 76.3975) (width 0.25) (layer B.Cu) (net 12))
 (segment (start 44.85 72) (end 45 72) (width 0.25) (layer F.Cu) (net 8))
 (via (at 45 72) (size 0.8) (drill 0.4) (layers F.Cu B.Cu) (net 8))
 (segment (start 45 72) (end 45 69) (width 0.25) (layer B.Cu) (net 8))
 (segment (start 45 72) (end 45 76.5) (width 0.25) (layer F.Cu) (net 8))
 (segment (start 45 76.5) (end 44.5 77) (width 0.25) (layer F.Cu) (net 8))
 (segment (start 44.5 77) (end 38.5 77) (width 0.25) (layer F.Cu) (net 8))
 (segment (start 38.5 77) (end 38 77.5) (width 0.25) (layer F.Cu) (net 8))
 (segment (start 38 77.5) (end 38 79) (width 0.25) (layer F.Cu) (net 8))
 (segment (start 38 79) (end 38 78.85) (width 0.25) (layer F.Cu) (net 8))
 (segment (start 38 80) (end 38 79) (width 0.25) (layer F.Cu) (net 8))
 (via (at 29 70) (size 0.8) (drill 0.4) (layers F.Cu B.Cu) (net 14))
 (segment (start 29.05 69.95) (end 29 70) (width 0.25) (layer B.Cu) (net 14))
 (segment (start 31 69.95) (end 29.05 69.95) (width 0.25) (layer B.Cu) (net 14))
 (segment (start 16.55 48.5) (end 15.62 47.57) (width 0.25) (layer F.Cu) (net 14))
 (segment (start 18.5 50) (end 17 48.5) (width 0.25) (layer F.Cu) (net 14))
 (segment (start 18.5 66) (end 18.5 50) (width 0.25) (layer F.Cu) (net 14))
 (segment (start 17 48.5) (end 16.55 48.5) (width 0.25) (layer F.Cu) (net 14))
 (segment (start 19 66.5) (end 18.5 66) (width 0.25) (layer F.Cu) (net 14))
 (segment (start 28 66.5) (end 19 66.5) (width 0.25) (layer F.Cu) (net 14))
 (segment (start 29 67.5) (end 28 66.5) (width 0.25) (layer F.Cu) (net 14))
 (segment (start 29 70) (end 29 67.5) (width 0.25) (layer F.Cu) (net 14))
 (via (at 35 70) (size 0.8) (drill 0.4) (layers F.Cu B.Cu) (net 11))
 (segment (start 35.05 69.95) (end 35 70) (width 0.25) (layer B.Cu) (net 11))
 (segment (start 37 69.95) (end 35.05 69.95) (width 0.25) (layer B.Cu) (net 11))
 (segment (start 30.5 70) (end 35 70) (width 0.25) (layer F.Cu) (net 11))
 (segment (start 29.5 67.36359) (end 29.5 69) (width 0.25) (layer F.Cu) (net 11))
 (segment (start 19 65.5) (end 19.5 66) (width 0.25) (layer F.Cu) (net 11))
 (segment (start 29.5 69) (end 30.5 70) (width 0.25) (layer F.Cu) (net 11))
 (segment (start 28.13641 66) (end 29.5 67.36359) (width 0.25) (layer F.Cu) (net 11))
 (segment (start 19.5 66) (end 28.13641 66) (width 0.25) (layer F.Cu) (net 11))
 (segment (start 19 48.5) (end 19 65.5) (width 0.25) (layer F.Cu) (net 11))
 (segment (start 19.009999 48.490001) (end 19 48.5) (width 0.25) (layer F.Cu) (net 11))
 (segment (start 19.009999 48.419999) (end 19.009999 48.490001) (width 0.25) (layer F.Cu) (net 11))
 (segment (start 18.16 47.57) (end 19.009999 48.419999) (width 0.25) (layer F.Cu) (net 11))
 (segment (start 43 69.95) (end 41.05 69.95) (width 0.25) (layer B.Cu) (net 9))
 (via (at 41 70) (size 0.8) (drill 0.4) (layers F.Cu B.Cu) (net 9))
 (segment (start 41.05 69.95) (end 41 70) (width 0.25) (layer B.Cu) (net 9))
 (segment (start 19.5 48.77) (end 20.7 47.57) (width 0.25) (layer F.Cu) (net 9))
 (segment (start 20 65.5) (end 19.5 65) (width 0.25) (layer F.Cu) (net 9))
 (segment (start 28.27282 65.5) (end 20 65.5) (width 0.25) (layer F.Cu) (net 9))
 (segment (start 29.95001 68.45001) (end 29.950009 67.177189) (width 0.25) (layer F.Cu) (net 9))
 (segment (start 29.950009 67.177189) (end 28.27282 65.5) (width 0.25) (layer F.Cu) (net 9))
 (segment (start 30.774999 69.274999) (end 29.95001 68.45001) (width 0.25) (layer F.Cu) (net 9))
 (segment (start 19.5 65) (end 19.5 48.77) (width 0.25) (layer F.Cu) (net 9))
 (segment (start 40.274999 69.274999) (end 30.774999 69.274999) (width 0.25) (layer F.Cu) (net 9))
 (segment (start 41 70) (end 40.274999 69.274999) (width 0.25) (layer F.Cu) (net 9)))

